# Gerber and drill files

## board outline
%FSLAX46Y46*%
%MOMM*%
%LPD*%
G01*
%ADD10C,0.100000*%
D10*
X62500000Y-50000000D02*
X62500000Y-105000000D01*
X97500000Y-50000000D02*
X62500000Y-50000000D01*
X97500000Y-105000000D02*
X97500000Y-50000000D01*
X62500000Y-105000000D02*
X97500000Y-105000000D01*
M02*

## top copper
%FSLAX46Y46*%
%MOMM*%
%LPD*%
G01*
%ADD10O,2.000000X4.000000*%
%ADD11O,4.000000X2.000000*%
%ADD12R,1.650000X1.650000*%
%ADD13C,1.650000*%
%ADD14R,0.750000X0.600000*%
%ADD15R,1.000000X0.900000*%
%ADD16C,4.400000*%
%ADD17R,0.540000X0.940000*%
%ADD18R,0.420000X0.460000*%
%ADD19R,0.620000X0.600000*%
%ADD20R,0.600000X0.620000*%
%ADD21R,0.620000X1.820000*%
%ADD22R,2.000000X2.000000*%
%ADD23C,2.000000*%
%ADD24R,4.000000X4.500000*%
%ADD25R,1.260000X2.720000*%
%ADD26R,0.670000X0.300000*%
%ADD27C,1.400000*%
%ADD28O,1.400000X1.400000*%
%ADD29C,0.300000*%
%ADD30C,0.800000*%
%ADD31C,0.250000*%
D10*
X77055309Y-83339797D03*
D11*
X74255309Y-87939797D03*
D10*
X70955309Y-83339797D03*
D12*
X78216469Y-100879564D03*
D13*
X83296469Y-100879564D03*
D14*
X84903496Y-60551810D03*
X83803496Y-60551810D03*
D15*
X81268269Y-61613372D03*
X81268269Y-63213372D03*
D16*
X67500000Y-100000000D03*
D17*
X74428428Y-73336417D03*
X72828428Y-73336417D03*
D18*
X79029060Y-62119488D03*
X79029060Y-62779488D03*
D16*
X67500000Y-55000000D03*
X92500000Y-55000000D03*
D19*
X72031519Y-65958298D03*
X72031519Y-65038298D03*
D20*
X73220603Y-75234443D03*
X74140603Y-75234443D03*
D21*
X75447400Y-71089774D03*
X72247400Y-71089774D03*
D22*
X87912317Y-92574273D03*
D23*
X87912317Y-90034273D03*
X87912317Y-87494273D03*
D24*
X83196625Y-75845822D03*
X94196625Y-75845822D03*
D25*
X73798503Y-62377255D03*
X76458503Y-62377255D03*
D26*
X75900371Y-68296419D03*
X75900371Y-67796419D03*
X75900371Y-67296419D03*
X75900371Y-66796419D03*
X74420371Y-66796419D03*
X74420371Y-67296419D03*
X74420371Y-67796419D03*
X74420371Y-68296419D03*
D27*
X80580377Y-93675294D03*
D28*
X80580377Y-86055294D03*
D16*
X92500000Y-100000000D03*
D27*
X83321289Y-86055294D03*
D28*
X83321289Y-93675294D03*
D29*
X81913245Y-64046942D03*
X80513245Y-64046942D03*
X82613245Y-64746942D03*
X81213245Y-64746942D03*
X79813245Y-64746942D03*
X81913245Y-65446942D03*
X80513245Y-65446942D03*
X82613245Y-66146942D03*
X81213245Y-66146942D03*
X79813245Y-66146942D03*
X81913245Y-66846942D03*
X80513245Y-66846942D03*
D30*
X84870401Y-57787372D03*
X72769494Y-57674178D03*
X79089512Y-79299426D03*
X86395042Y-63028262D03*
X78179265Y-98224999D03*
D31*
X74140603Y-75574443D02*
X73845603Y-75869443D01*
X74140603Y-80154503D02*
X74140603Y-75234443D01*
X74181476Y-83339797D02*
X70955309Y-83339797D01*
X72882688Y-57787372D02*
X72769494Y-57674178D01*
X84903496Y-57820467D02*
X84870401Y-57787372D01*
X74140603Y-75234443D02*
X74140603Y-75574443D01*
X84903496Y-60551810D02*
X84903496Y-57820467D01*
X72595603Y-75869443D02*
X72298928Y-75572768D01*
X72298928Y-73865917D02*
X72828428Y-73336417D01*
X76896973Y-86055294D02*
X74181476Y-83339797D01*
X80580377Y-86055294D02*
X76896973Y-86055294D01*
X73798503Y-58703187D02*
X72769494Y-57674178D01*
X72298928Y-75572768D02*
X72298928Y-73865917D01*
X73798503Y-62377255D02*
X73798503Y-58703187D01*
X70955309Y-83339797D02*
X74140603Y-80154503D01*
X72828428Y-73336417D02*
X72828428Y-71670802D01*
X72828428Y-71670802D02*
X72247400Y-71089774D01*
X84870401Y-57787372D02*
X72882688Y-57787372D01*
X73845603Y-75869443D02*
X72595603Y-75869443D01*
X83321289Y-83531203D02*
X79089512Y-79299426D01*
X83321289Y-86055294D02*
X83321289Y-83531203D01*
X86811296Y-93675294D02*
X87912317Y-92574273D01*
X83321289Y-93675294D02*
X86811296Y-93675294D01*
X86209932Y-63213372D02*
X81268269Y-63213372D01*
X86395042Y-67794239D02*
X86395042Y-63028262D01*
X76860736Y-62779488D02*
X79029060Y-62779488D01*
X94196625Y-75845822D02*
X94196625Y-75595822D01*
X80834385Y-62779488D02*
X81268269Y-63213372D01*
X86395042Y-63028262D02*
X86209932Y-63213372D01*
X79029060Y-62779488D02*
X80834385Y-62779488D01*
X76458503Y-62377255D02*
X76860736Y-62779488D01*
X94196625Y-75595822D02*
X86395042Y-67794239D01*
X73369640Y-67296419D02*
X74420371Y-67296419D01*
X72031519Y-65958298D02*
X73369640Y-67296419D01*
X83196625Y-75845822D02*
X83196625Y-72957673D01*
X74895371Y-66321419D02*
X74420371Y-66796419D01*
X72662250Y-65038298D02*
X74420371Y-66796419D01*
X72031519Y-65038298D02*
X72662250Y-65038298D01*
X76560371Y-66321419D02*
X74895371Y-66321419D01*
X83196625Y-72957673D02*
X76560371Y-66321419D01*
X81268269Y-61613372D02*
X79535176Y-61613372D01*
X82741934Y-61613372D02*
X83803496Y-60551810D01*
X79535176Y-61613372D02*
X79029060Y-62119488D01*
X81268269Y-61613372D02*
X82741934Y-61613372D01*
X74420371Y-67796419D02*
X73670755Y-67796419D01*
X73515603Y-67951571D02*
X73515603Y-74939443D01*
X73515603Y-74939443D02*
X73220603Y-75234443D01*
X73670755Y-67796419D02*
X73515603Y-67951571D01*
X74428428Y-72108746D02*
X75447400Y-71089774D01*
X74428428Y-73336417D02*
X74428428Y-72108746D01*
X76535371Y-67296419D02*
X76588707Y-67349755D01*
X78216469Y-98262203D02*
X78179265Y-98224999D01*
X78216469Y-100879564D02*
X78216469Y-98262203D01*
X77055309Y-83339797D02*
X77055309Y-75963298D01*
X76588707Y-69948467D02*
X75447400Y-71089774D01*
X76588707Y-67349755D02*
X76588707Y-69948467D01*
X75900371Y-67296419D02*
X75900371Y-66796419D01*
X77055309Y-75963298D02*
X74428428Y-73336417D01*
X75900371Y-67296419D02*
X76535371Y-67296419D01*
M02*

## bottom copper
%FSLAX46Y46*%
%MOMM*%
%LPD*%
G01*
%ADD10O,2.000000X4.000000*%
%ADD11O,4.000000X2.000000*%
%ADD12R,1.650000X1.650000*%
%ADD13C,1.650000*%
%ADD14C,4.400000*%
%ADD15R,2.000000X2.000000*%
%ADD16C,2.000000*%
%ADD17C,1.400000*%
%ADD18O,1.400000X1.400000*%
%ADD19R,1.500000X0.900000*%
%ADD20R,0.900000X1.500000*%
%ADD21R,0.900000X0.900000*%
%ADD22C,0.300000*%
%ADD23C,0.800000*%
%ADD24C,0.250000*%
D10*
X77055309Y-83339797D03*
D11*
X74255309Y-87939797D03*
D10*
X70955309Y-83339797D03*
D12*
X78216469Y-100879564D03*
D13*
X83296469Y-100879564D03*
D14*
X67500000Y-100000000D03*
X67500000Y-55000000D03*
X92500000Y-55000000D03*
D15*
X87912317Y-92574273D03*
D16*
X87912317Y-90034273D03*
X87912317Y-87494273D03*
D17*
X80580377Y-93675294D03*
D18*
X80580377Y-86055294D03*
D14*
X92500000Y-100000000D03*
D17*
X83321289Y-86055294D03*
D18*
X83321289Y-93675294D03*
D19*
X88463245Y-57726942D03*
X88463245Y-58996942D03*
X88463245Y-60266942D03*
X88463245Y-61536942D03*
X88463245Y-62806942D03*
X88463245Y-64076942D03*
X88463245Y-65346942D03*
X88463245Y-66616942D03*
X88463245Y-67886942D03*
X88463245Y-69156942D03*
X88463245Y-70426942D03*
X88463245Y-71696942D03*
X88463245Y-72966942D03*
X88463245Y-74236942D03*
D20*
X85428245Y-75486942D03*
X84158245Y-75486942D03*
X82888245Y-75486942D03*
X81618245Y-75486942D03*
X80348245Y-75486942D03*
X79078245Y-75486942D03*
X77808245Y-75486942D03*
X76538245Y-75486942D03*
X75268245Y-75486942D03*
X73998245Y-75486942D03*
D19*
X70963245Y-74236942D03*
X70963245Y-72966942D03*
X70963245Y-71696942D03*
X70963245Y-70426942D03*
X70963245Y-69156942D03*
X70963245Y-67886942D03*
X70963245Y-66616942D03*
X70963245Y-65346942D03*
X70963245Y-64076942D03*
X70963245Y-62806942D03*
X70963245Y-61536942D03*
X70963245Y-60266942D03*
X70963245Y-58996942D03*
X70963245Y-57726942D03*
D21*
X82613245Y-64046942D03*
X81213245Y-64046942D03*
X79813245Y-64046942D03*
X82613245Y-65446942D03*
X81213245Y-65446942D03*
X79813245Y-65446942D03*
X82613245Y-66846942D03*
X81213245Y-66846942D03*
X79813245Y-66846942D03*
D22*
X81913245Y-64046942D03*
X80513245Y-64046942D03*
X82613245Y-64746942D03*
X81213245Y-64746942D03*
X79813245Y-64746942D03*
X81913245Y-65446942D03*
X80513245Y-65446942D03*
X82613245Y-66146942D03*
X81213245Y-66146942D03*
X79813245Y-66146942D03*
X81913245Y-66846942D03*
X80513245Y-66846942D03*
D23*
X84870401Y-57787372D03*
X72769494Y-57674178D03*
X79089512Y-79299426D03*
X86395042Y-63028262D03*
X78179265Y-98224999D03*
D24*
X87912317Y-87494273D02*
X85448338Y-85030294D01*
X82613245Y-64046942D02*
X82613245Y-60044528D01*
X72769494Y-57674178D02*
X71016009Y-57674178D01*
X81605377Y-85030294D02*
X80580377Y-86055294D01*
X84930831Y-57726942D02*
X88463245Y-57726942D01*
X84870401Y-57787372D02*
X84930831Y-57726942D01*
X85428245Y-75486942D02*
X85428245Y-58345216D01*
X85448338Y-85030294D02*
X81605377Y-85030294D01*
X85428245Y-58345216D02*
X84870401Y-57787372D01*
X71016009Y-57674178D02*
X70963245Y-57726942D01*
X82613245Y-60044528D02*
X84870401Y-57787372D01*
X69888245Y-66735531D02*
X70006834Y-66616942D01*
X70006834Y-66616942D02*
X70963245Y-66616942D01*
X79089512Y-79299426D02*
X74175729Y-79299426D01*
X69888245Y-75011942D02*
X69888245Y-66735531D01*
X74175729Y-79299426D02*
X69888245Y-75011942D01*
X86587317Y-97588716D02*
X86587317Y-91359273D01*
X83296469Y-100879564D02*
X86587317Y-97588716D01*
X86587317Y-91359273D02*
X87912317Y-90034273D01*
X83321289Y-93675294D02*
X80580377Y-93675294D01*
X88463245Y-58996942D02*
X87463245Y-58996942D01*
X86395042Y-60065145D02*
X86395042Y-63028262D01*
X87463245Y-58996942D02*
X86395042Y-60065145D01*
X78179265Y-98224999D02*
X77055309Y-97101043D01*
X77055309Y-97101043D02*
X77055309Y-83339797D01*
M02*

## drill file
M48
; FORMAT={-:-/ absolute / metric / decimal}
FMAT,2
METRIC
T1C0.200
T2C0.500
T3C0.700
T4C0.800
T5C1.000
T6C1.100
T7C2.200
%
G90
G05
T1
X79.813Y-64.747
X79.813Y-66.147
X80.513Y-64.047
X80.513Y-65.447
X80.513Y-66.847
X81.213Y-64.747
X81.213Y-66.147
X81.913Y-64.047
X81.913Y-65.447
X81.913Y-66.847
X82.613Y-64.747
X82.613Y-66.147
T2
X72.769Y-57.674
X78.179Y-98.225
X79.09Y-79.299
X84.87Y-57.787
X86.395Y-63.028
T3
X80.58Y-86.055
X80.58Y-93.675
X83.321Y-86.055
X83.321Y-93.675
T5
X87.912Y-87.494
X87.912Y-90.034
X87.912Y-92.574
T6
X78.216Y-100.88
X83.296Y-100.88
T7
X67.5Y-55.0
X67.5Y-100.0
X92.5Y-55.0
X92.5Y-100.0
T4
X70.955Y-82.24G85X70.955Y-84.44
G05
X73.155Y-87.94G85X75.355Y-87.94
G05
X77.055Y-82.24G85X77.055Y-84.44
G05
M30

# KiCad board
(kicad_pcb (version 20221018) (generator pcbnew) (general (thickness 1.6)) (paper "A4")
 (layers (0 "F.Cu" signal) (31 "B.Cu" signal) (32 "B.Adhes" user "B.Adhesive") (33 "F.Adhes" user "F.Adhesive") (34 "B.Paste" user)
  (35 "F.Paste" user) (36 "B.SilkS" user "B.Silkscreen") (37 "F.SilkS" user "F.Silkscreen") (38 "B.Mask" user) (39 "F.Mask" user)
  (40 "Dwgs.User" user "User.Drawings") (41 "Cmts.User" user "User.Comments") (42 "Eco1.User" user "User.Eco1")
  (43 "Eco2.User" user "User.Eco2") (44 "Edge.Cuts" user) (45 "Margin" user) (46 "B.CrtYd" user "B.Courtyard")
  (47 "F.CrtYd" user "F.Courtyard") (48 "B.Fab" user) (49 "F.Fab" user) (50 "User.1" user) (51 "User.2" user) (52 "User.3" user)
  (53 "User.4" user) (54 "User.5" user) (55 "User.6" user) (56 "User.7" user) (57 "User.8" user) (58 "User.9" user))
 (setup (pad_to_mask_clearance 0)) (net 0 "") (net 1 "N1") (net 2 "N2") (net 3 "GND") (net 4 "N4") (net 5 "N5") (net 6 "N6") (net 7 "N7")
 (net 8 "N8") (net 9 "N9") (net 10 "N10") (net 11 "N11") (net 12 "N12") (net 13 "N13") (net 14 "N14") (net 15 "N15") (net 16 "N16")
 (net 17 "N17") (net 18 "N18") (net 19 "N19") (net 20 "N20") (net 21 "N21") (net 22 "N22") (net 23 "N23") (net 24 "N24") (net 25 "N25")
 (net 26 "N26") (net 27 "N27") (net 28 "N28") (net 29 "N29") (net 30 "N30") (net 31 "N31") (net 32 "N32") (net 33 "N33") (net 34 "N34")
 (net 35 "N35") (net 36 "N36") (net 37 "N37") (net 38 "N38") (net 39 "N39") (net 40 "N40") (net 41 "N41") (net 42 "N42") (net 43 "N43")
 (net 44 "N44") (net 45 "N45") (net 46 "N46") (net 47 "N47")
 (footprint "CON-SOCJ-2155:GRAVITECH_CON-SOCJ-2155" (layer "F.Cu") (at 70.955309 83.339797)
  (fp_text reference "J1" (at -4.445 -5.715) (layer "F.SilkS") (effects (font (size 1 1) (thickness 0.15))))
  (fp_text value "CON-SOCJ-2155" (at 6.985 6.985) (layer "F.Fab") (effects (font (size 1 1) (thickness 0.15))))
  (pad "1" thru_hole oval (at 6.1 0) (size 2 4) (drill oval 0.8 3) (layers "*.Cu" "*.Mask") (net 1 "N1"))
  (pad "2" thru_hole oval (at 3.3 4.6) (size 4 2) (drill oval 3 0.8) (layers "*.Cu" "*.Mask") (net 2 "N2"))
  (pad "3" thru_hole oval (at 0 0) (size 2 4) (drill oval 0.8 3) (layers "*.Cu" "*.Mask") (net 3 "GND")))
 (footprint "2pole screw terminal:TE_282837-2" (layer "F.Cu") (at 80.756469 100.879564)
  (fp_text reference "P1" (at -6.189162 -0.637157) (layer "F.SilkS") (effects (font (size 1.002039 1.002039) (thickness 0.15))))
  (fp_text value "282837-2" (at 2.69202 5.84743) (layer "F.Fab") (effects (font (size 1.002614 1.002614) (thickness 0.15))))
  (pad "1" thru_hole rect (at -2.54 0) (size 1.65 1.65) (drill 1.1) (layers "*.Cu" "*.Mask") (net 1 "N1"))
  (pad "2" thru_hole circle (at 2.54 0) (size 1.65 1.65) (drill 1.1) (layers "*.Cu" "*.Mask") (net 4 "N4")))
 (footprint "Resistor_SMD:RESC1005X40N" (layer "F.Cu") (at 84.353496 60.55181 180)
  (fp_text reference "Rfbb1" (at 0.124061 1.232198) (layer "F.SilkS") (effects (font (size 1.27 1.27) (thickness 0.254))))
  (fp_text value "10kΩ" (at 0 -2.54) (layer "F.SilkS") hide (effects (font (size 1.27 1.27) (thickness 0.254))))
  (pad "1" smd rect (at -0.55 0 270) (size 0.6 0.75) (layers "F.Cu" "F.Paste" "F.Mask") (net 3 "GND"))
  (pad "2" smd rect (at 0.55 0 270) (size 0.6 0.75) (layers "F.Cu" "F.Paste" "F.Mask") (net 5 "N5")))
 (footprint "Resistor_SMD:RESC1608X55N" (layer "F.Cu") (at 81.268269 62.413372 -90)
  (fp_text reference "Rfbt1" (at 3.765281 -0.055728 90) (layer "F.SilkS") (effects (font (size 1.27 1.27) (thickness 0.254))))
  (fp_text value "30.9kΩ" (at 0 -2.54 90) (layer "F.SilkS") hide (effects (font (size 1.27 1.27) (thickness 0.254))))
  (pad "1" smd rect (at -0.8 0 270) (size 0.9 1) (layers "F.Cu" "F.Paste" "F.Mask") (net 5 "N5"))
  (pad "2" smd rect (at 0.8 0 270) (size 0.9 1) (layers "F.Cu" "F.Paste" "F.Mask") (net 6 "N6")))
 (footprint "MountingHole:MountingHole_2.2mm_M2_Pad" (layer "F.Cu") (at 67.5 100)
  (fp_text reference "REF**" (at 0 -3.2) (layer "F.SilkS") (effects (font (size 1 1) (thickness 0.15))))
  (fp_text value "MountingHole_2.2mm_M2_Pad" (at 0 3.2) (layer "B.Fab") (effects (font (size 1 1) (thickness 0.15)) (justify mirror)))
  (pad "1" thru_hole circle (at 0 0) (size 4.4 4.4) (drill 2.2) (layers "*.Cu" "*.Mask")))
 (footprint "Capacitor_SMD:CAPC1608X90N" (layer "F.Cu") (at 73.628428 73.336417 180)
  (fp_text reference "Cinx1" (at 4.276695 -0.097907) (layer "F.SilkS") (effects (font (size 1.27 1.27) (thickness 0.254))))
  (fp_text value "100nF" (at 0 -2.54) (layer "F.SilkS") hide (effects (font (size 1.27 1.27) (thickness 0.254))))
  (pad "1" smd rect (at -0.8 0 180) (size 0.54 0.94) (layers "F.Cu" "F.Paste" "F.Mask") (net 1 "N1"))
  (pad "2" smd rect (at 0.8 0 180) (size 0.54 0.94) (layers "F.Cu" "F.Paste" "F.Mask") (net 3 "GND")))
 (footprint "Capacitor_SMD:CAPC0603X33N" (layer "F.Cu") (at 79.02906 62.449488 -90)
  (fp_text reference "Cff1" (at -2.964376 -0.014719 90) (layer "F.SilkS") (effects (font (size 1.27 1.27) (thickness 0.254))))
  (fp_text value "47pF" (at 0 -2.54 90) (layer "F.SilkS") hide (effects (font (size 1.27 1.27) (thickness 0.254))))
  (pad "1" smd rect (at -0.33 0) (size 0.42 0.46) (layers "F.Cu" "F.Paste" "F.Mask") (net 5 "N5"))
  (pad "2" smd rect (at 0.33 0) (size 0.42 0.46) (layers "F.Cu" "F.Paste" "F.Mask") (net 6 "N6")))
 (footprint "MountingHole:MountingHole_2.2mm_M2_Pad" (layer "F.Cu") (at 67.5 55)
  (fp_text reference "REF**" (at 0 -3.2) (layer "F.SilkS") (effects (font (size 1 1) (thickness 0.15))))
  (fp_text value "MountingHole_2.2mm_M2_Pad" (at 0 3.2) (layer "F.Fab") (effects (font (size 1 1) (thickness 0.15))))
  (pad "1" thru_hole circle (at 0 0) (size 4.4 4.4) (drill 2.2) (layers "*.Cu" "*.Mask")))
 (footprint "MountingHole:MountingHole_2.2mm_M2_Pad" (layer "F.Cu") (at 92.5 55)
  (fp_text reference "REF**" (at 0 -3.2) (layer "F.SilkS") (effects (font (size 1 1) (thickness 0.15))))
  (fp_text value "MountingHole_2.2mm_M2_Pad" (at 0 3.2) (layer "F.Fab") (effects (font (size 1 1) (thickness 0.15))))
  (pad "1" thru_hole circle (at 0 0) (size 4.4 4.4) (drill 2.2) (layers "*.Cu" "*.Mask")))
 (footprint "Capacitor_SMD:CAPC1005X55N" (layer "F.Cu") (at 72.031519 65.498298 90)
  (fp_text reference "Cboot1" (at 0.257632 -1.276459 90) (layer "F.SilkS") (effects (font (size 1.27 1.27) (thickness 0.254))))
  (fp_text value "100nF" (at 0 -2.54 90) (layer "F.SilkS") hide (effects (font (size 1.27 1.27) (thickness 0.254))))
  (pad "1" smd rect (at -0.46 0 90) (size 0.6 0.62) (layers "F.Cu" "F.Paste" "F.Mask") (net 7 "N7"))
  (pad "2" smd rect (at 0.46 0 90) (size 0.6 0.62) (layers "F.Cu" "F.Paste" "F.Mask") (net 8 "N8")))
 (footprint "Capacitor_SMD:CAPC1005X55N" (layer "F.Cu") (at 73.680603 75.234443)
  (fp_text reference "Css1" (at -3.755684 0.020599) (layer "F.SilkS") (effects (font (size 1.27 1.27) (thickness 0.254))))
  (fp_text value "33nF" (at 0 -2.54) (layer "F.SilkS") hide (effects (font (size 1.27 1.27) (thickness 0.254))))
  (pad "1" smd rect (at -0.46 0) (size 0.6 0.62) (layers "F.Cu" "F.Paste" "F.Mask") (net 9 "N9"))
  (pad "2" smd rect (at 0.46 0) (size 0.6 0.62) (layers "F.Cu" "F.Paste" "F.Mask") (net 3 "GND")))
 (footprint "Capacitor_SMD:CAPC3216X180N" (layer "F.Cu") (at 73.8474 71.089774 180)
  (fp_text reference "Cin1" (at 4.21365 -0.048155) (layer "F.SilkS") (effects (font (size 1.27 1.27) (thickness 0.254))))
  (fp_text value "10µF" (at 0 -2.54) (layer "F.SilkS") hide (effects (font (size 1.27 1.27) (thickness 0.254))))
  (pad "1" smd rect (at -1.6 0 180) (size 0.62 1.82) (layers "F.Cu" "F.Paste" "F.Mask") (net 1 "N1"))
  (pad "2" smd rect (at 1.6 0 180) (size 0.62 1.82) (layers "F.Cu" "F.Paste" "F.Mask") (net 3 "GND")))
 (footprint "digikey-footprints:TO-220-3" (layer "F.Cu") (at 87.912317 92.574273 90)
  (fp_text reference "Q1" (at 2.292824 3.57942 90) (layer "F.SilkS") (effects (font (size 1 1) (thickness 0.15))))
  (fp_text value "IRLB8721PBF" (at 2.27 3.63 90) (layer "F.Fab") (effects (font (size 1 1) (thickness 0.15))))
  (pad "1" thru_hole rect (at 0 0 90) (size 2 2) (drill 1) (layers "*.Cu" "*.Mask") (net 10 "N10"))
  (pad "2" thru_hole circle (at 2.54 0 90) (size 2 2) (drill 1) (layers "*.Cu" "*.Mask") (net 4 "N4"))
  (pad "3" thru_hole circle (at 5.08 0 90) (size 2 2) (drill 1) (layers "*.Cu" "*.Mask") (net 3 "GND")))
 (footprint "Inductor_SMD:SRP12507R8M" (layer "F.Cu") (at 88.696625 75.845822)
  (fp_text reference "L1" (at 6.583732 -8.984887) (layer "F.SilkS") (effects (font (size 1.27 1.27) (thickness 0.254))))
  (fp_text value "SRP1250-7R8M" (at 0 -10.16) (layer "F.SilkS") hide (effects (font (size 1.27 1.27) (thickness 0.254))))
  (pad "1" smd rect (at -5.5 0) (size 4 4.5) (layers "F.Cu" "F.Paste" "F.Mask") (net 8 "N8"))
  (pad "2" smd rect (at 5.5 0) (size 4 4.5) (layers "F.Cu" "F.Paste" "F.Mask") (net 6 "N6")))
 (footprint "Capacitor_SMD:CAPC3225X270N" (layer "F.Cu") (at 75.128503 62.377255)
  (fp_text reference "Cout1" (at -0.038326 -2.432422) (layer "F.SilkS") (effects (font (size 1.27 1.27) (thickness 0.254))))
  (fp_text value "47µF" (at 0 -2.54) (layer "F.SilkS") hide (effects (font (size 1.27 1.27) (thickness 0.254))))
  (pad "1" smd rect (at -1.33 0) (size 1.26 2.72) (layers "F.Cu" "F.Paste" "F.Mask") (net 3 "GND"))
  (pad "2" smd rect (at 1.33 0) (size 1.26 2.72) (layers "F.Cu" "F.Paste" "F.Mask") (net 6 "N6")))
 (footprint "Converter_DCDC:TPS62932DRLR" (layer "F.Cu") (at 75.160371 67.546419 180)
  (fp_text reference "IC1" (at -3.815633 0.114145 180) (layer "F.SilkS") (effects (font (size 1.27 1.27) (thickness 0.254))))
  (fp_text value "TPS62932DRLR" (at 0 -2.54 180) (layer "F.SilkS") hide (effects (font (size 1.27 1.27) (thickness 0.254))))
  (pad "1" smd rect (at -0.74 -0.75 270) (size 0.3 0.67) (layers "F.Cu" "F.Paste" "F.Mask") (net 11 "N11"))
  (pad "2" smd rect (at -0.74 -0.25 270) (size 0.3 0.67) (layers "F.Cu" "F.Paste" "F.Mask") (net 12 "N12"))
  (pad "3" smd rect (at -0.74 0.25 270) (size 0.3 0.67) (layers "F.Cu" "F.Paste" "F.Mask") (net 1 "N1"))
  (pad "4" smd rect (at -0.74 0.75 270) (size 0.3 0.67) (layers "F.Cu" "F.Paste" "F.Mask") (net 1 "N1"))
  (pad "5" smd rect (at 0.74 0.75 270) (size 0.3 0.67) (layers "F.Cu" "F.Paste" "F.Mask") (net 8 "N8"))
  (pad "6" smd rect (at 0.74 0.25 270) (size 0.3 0.67) (layers "F.Cu" "F.Paste" "F.Mask") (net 7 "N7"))
  (pad "7" smd rect (at 0.74 -0.25 270) (size 0.3 0.67) (layers "F.Cu" "F.Paste" "F.Mask") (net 9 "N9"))
  (pad "8" smd rect (at 0.74 -0.75 270) (size 0.3 0.67) (layers "F.Cu" "F.Paste" "F.Mask") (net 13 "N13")))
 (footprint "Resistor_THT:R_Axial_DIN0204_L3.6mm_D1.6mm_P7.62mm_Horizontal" (layer "F.Cu") (at 80.580377 93.675294 90)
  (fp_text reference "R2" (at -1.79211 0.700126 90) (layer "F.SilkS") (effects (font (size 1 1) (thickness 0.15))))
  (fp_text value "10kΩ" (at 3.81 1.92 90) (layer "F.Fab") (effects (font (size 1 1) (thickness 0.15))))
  (pad "1" thru_hole circle (at 0 0 90) (size 1.4 1.4) (drill 0.7) (layers "*.Cu" "*.Mask") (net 10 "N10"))
  (pad "2" thru_hole oval (at 7.62 0 90) (size 1.4 1.4) (drill 0.7) (layers "*.Cu" "*.Mask") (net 3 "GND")))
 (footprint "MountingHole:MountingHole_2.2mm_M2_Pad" (layer "F.Cu") (at 92.5 100)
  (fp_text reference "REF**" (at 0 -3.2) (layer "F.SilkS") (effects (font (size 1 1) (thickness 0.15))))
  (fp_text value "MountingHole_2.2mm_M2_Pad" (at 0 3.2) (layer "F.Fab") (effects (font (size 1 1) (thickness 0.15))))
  (pad "1" thru_hole circle (at 0 0) (size 4.4 4.4) (drill 2.2) (layers "*.Cu" "*.Mask")))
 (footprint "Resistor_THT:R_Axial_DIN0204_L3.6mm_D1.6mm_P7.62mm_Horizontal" (layer "F.Cu") (at 83.321289 86.055294 -90)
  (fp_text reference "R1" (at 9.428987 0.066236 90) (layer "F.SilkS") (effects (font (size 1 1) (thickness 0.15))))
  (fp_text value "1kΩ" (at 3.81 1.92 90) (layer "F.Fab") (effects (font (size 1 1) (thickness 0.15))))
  (pad "1" thru_hole circle (at 0 0 270) (size 1.4 1.4) (drill 0.7) (layers "*.Cu" "*.Mask") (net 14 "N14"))
  (pad "2" thru_hole oval (at 7.62 0 270) (size 1.4 1.4) (drill 0.7) (layers "*.Cu" "*.Mask") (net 10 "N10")))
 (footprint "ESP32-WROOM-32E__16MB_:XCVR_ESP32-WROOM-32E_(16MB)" (layer "B.Cu") (at 79.713245 62.986942 180)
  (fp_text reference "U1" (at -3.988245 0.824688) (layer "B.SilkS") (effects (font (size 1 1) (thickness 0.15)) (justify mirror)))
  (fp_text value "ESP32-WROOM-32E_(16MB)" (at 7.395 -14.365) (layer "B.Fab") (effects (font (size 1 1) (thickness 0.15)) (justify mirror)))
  (pad "1" smd rect (at -8.75 5.26 180) (size 1.5 0.9) (layers "B.Cu" "B.Paste" "B.Mask") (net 3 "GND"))
  (pad "2" smd rect (at -8.75 3.99 180) (size 1.5 0.9) (layers "B.Cu" "B.Paste" "B.Mask") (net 6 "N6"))
  (pad "3" smd rect (at -8.75 2.72 180) (size 1.5 0.9) (layers "B.Cu" "B.Paste" "B.Mask") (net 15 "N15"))
  (pad "4" smd rect (at -8.75 1.45 180) (size 1.5 0.9) (layers "B.Cu" "B.Paste" "B.Mask") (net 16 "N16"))
  (pad "5" smd rect (at -8.75 0.18 180) (size 1.5 0.9) (layers "B.Cu" "B.Paste" "B.Mask") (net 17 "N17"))
  (pad "6" smd rect (at -8.75 -1.09 180) (size 1.5 0.9) (layers "B.Cu" "B.Paste" "B.Mask") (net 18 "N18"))
  (pad "7" smd rect (at -8.75 -2.36 180) (size 1.5 0.9) (layers "B.Cu" "B.Paste" "B.Mask") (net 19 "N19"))
  (pad "8" smd rect (at -8.75 -3.63 180) (size 1.5 0.9) (layers "B.Cu" "B.Paste" "B.Mask") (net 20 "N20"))
  (pad "9" smd rect (at -8.75 -4.9 180) (size 1.5 0.9) (layers "B.Cu" "B.Paste" "B.Mask") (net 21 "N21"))
  (pad "10" smd rect (at -8.75 -6.17 180) (size 1.5 0.9) (layers "B.Cu" "B.Paste" "B.Mask") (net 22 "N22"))
  (pad "11" smd rect (at -8.75 -7.44 180) (size 1.5 0.9) (layers "B.Cu" "B.Paste" "B.Mask") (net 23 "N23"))
  (pad "12" smd rect (at -8.75 -8.71 180) (size 1.5 0.9) (layers "B.Cu" "B.Paste" "B.Mask") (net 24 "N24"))
  (pad "13" smd rect (at -8.75 -9.98 180) (size 1.5 0.9) (layers "B.Cu" "B.Paste" "B.Mask") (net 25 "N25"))
  (pad "14" smd rect (at -8.75 -11.25 180) (size 1.5 0.9) (layers "B.Cu" "B.Paste" "B.Mask") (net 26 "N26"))
  (pad "15" smd rect (at -5.715 -12.5 180) (size 0.9 1.5) (layers "B.Cu" "B.Paste" "B.Mask") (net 3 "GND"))
  (pad "16" smd rect (at -4.445 -12.5 180) (size 0.9 1.5) (layers "B.Cu" "B.Paste" "B.Mask") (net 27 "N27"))
  (pad "17" smd rect (at -3.175 -12.5 180) (size 0.9 1.5) (layers "B.Cu" "B.Paste" "B.Mask") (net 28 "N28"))
  (pad "18" smd rect (at -1.905 -12.5 180) (size 0.9 1.5) (layers "B.Cu" "B.Paste" "B.Mask") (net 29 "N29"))
  (pad "19" smd rect (at -0.635 -12.5 180) (size 0.9 1.5) (layers "B.Cu" "B.Paste" "B.Mask") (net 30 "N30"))
  (pad "20" smd rect (at 0.635 -12.5 180) (size 0.9 1.5) (layers "B.Cu" "B.Paste" "B.Mask") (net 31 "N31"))
  (pad "21" smd rect (at 1.905 -12.5 180) (size 0.9 1.5) (layers "B.Cu" "B.Paste" "B.Mask") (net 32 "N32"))
  (pad "22" smd rect (at 3.175 -12.5 180) (size 0.9 1.5) (layers "B.Cu" "B.Paste" "B.Mask") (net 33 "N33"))
  (pad "23" smd rect (at 4.445 -12.5 180) (size 0.9 1.5) (layers "B.Cu" "B.Paste" "B.Mask") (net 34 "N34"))
  (pad "24" smd rect (at 5.715 -12.5 180) (size 0.9 1.5) (layers "B.Cu" "B.Paste" "B.Mask") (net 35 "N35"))
  (pad "25" smd rect (at 8.75 -11.25 180) (size 1.5 0.9) (layers "B.Cu" "B.Paste" "B.Mask") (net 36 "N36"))
  (pad "26" smd rect (at 8.75 -9.98 180) (size 1.5 0.9) (layers "B.Cu" "B.Paste" "B.Mask") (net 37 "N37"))
  (pad "27" smd rect (at 8.75 -8.71 180) (size 1.5 0.9) (layers "B.Cu" "B.Paste" "B.Mask") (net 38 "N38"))
  (pad "28" smd rect (at 8.75 -7.44 180) (size 1.5 0.9) (layers "B.Cu" "B.Paste" "B.Mask") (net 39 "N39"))
  (pad "29" smd rect (at 8.75 -6.17 180) (size 1.5 0.9) (layers "B.Cu" "B.Paste" "B.Mask") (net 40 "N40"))
  (pad "30" smd rect (at 8.75 -4.9 180) (size 1.5 0.9) (layers "B.Cu" "B.Paste" "B.Mask") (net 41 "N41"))
  (pad "31" smd rect (at 8.75 -3.63 180) (size 1.5 0.9) (layers "B.Cu" "B.Paste" "B.Mask") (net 14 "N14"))
  (pad "32" smd rect (at 8.75 -2.36 180) (size 1.5 0.9) (layers "B.Cu" "B.Paste" "B.Mask") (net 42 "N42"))
  (pad "33" smd rect (at 8.75 -1.09 180) (size 1.5 0.9) (layers "B.Cu" "B.Paste" "B.Mask") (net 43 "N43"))
  (pad "34" smd rect (at 8.75 0.18 180) (size 1.5 0.9) (layers "B.Cu" "B.Paste" "B.Mask") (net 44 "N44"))
  (pad "35" smd rect (at 8.75 1.45 180) (size 1.5 0.9) (layers "B.Cu" "B.Paste" "B.Mask") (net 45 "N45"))
  (pad "36" smd rect (at 8.75 2.72 180) (size 1.5 0.9) (layers "B.Cu" "B.Paste" "B.Mask") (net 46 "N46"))
  (pad "37" smd rect (at 8.75 3.99 180) (size 1.5 0.9) (layers "B.Cu" "B.Paste" "B.Mask") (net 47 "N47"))
  (pad "38" smd rect (at 8.75 5.26 180) (size 1.5 0.9) (layers "B.Cu" "B.Paste" "B.Mask") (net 3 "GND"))
  (pad "39_1" smd rect (at -2.9 -1.06 180) (size 0.9 0.9) (layers "B.Cu" "B.Paste" "B.Mask") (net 3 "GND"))
  (pad "39_2" smd rect (at -1.5 -1.06 180) (size 0.9 0.9) (layers "B.Cu" "B.Paste" "B.Mask") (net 3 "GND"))
  (pad "39_3" smd rect (at -0.1 -1.06 180) (size 0.9 0.9) (layers "B.Cu" "B.Paste" "B.Mask") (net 3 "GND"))
  (pad "39_4" smd rect (at -2.9 -2.46 180) (size 0.9 0.9) (layers "B.Cu" "B.Paste" "B.Mask") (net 3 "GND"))
  (pad "39_5" smd rect (at -1.5 -2.46 180) (size 0.9 0.9) (layers "B.Cu" "B.Paste" "B.Mask") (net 3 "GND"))
  (pad "39_6" smd rect (at -0.1 -2.46 180) (size 0.9 0.9) (layers "B.Cu" "B.Paste" "B.Mask") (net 3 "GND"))
  (pad "39_7" smd rect (at -2.9 -3.86 180) (size 0.9 0.9) (layers "B.Cu" "B.Paste" "B.Mask") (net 3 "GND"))
  (pad "39_8" smd rect (at -1.5 -3.86 180) (size 0.9 0.9) (layers "B.Cu" "B.Paste" "B.Mask") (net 3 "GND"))
  (pad "39_9" smd rect (at -0.1 -3.86 180) (size 0.9 0.9) (layers "B.Cu" "B.Paste" "B.Mask") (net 3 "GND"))
  (pad "39_10" thru_hole circle (at -2.2 -1.06 180) (size 0.3 0.3) (drill 0.2) (layers "*.Cu"))
  (pad "39_11" thru_hole circle (at -0.8 -1.06 180) (size 0.3 0.3) (drill 0.2) (layers "*.Cu"))
  (pad "39_12" thru_hole circle (at -2.9 -1.76 180) (size 0.3 0.3) (drill 0.2) (layers "*.Cu"))
  (pad "39_13" thru_hole circle (at -1.5 -1.76 180) (size 0.3 0.3) (drill 0.2) (layers "*.Cu"))
  (pad "39_14" thru_hole circle (at -0.1 -1.76 180) (size 0.3 0.3) (drill 0.2) (layers "*.Cu"))
  (pad "39_15" thru_hole circle (at -2.2 -2.46 180) (size 0.3 0.3) (drill 0.2) (layers "*.Cu"))
  (pad "39_16" thru_hole circle (at -0.8 -2.46 180) (size 0.3 0.3) (drill 0.2) (layers "*.Cu"))
  (pad "39_17" thru_hole circle (at -2.9 -3.16 180) (size 0.3 0.3) (drill 0.2) (layers "*.Cu"))
  (pad "39_18" thru_hole circle (at -1.5 -3.16 180) (size 0.3 0.3) (drill 0.2) (layers "*.Cu"))
  (pad "39_19" thru_hole circle (at -0.1 -3.16 180) (size 0.3 0.3) (drill 0.2) (layers "*.Cu"))
  (pad "39_20" thru_hole circle (at -2.2 -3.86 180) (size 0.3 0.3) (drill 0.2) (layers "*.Cu"))
  (pad "39_21" thru_hole circle (at -0.8 -3.86 180) (size 0.3 0.3) (drill 0.2) (layers "*.Cu"))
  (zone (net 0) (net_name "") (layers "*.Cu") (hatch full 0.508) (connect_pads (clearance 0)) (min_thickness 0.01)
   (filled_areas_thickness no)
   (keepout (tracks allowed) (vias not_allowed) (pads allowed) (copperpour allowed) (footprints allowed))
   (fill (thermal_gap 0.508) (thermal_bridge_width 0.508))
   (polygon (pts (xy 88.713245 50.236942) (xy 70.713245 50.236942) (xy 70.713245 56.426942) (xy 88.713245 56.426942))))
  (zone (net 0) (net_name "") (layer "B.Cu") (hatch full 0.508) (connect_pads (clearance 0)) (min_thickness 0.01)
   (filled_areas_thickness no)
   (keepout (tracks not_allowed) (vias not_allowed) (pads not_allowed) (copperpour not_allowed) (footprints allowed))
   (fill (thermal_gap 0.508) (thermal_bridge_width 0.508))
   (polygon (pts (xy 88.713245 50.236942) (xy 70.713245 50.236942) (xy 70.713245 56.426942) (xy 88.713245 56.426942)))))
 (gr_line (start 62.5 50) (end 62.5 105) (stroke (width 0.1) (type default)) (layer "Edge.Cuts"))
 (gr_line (start 97.5 50) (end 62.5 50) (stroke (width 0.1) (type default)) (layer "Edge.Cuts"))
 (gr_line (start 97.5 105) (end 97.5 50) (stroke (width 0.1) (type default)) (layer "Edge.Cuts"))
 (gr_line (start 62.5 105) (end 97.5 105) (stroke (width 0.1) (type default)) (layer "Edge.Cuts"))
 (segment (start 74.140603 75.574443) (end 73.845603 75.869443) (width 0.25) (layer "F.Cu") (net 3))
 (segment (start 74.140603 80.154503) (end 74.140603 75.234443) (width 0.25) (layer "F.Cu") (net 3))
 (segment (start 74.181476 83.339797) (end 70.955309 83.339797) (width 0.25) (layer "F.Cu") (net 3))
 (segment (start 72.882688 57.787372) (end 72.769494 57.674178) (width 0.25) (layer "F.Cu") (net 3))
 (segment (start 84.903496 57.820467) (end 84.870401 57.787372) (width 0.25) (layer "F.Cu") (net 3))
 (segment (start 74.140603 75.234443) (end 74.140603 75.574443) (width 0.25) (layer "F.Cu") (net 3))
 (segment (start 84.903496 60.55181) (end 84.903496 57.820467) (width 0.25) (layer "F.Cu") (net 3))
 (segment (start 72.595603 75.869443) (end 72.298928 75.572768) (width 0.25) (layer "F.Cu") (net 3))
 (segment (start 72.298928 73.865917) (end 72.828428 73.336417) (width 0.25) (layer "F.Cu") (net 3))
 (segment (start 76.896973 86.055294) (end 74.181476 83.339797) (width 0.25) (layer "F.Cu") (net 3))
 (segment (start 80.580377 86.055294) (end 76.896973 86.055294) (width 0.25) (layer "F.Cu") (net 3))
 (segment (start 73.798503 58.703187) (end 72.769494 57.674178) (width 0.25) (layer "F.Cu") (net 3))
 (segment (start 72.298928 75.572768) (end 72.298928 73.865917) (width 0.25) (layer "F.Cu") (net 3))
 (segment (start 73.798503 62.377255) (end 73.798503 58.703187) (width 0.25) (layer "F.Cu") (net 3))
 (segment (start 70.955309 83.339797) (end 74.140603 80.154503) (width 0.25) (layer "F.Cu") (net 3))
 (segment (start 72.828428 73.336417) (end 72.828428 71.670802) (width 0.25) (layer "F.Cu") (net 3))
 (segment (start 72.828428 71.670802) (end 72.2474 71.089774) (width 0.25) (layer "F.Cu") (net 3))
 (segment (start 84.870401 57.787372) (end 72.882688 57.787372) (width 0.25) (layer "F.Cu") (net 3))
 (segment (start 73.845603 75.869443) (end 72.595603 75.869443) (width 0.25) (layer "F.Cu") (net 3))
 (via (at 84.870401 57.787372) (size 0.8) (drill 0.5) (layers "F.Cu" "B.Cu") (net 3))
 (via (at 72.769494 57.674178) (size 0.8) (drill 0.5) (layers "F.Cu" "B.Cu") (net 3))
 (segment (start 87.912317 87.494273) (end 85.448338 85.030294) (width 0.25) (layer "B.Cu") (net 3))
 (segment (start 82.613245 64.046942) (end 82.613245 60.044528) (width 0.25) (layer "B.Cu") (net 3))
 (segment (start 72.769494 57.674178) (end 71.016009 57.674178) (width 0.25) (layer "B.Cu") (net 3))
 (segment (start 81.605377 85.030294) (end 80.580377 86.055294) (width 0.25) (layer "B.Cu") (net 3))
 (segment (start 84.930831 57.726942) (end 88.463245 57.726942) (width 0.25) (layer "B.Cu") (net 3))
 (segment (start 84.870401 57.787372) (end 84.930831 57.726942) (width 0.25) (layer "B.Cu") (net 3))
 (segment (start 85.428245 75.486942) (end 85.428245 58.345216) (width 0.25) (layer "B.Cu") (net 3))
 (segment (start 85.448338 85.030294) (end 81.605377 85.030294) (width 0.25) (layer "B.Cu") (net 3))
 (segment (start 85.428245 58.345216) (end 84.870401 57.787372) (width 0.25) (layer "B.Cu") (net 3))
 (segment (start 71.016009 57.674178) (end 70.963245 57.726942) (width 0.25) (layer "B.Cu") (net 3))
 (segment (start 82.613245 60.044528) (end 84.870401 57.787372) (width 0.25) (layer "B.Cu") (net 3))
 (segment (start 83.321289 83.531203) (end 79.089512 79.299426) (width 0.25) (layer "F.Cu") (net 14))
 (segment (start 83.321289 86.055294) (end 83.321289 83.531203) (width 0.25) (layer "F.Cu") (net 14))
 (via (at 79.089512 79.299426) (size 0.8) (drill 0.5) (layers "F.Cu" "B.Cu") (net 14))
 (segment (start 69.888245 66.735531) (end 70.006834 66.616942) (width 0.25) (layer "B.Cu") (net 14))
 (segment (start 70.006834 66.616942) (end 70.963245 66.616942) (width 0.25) (layer "B.Cu") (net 14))
 (segment (start 79.089512 79.299426) (end 74.175729 79.299426) (width 0.25) (layer "B.Cu") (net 14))
 (segment (start 69.888245 75.011942) (end 69.888245 66.735531) (width 0.25) (layer "B.Cu") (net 14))
 (segment (start 74.175729 79.299426) (end 69.888245 75.011942) (width 0.25) (layer "B.Cu") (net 14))
 (segment (start 86.587317 97.588716) (end 86.587317 91.359273) (width 0.25) (layer "B.Cu") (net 4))
 (segment (start 83.296469 100.879564) (end 86.587317 97.588716) (width 0.25) (layer "B.Cu") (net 4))
 (segment (start 86.587317 91.359273) (end 87.912317 90.034273) (width 0.25) (layer "B.Cu") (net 4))
 (segment (start 86.811296 93.675294) (end 87.912317 92.574273) (width 0.25) (layer "F.Cu") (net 10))
 (segment (start 83.321289 93.675294) (end 86.811296 93.675294) (width 0.25) (layer "F.Cu") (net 10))
 (segment (start 83.321289 93.675294) (end 80.580377 93.675294) (width 0.25) (layer "B.Cu") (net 10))
 (segment (start 86.209932 63.213372) (end 81.268269 63.213372) (width 0.25) (layer "F.Cu") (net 6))
 (segment (start 86.395042 67.794239) (end 86.395042 63.028262) (width 0.25) (layer "F.Cu") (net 6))
 (segment (start 76.860736 62.779488) (end 79.02906 62.779488) (width 0.25) (layer "F.Cu") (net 6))
 (segment (start 94.196625 75.845822) (end 94.196625 75.595822) (width 0.25) (layer "F.Cu") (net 6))
 (segment (start 80.834385 62.779488) (end 81.268269 63.213372) (width 0.25) (layer "F.Cu") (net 6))
 (segment (start 86.395042 63.028262) (end 86.209932 63.213372) (width 0.25) (layer "F.Cu") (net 6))
 (segment (start 79.02906 62.779488) (end 80.834385 62.779488) (width 0.25) (layer "F.Cu") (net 6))
 (segment (start 76.458503 62.377255) (end 76.860736 62.779488) (width 0.25) (layer "F.Cu") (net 6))
 (segment (start 94.196625 75.595822) (end 86.395042 67.794239) (width 0.25) (layer "F.Cu") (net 6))
 (via (at 86.395042 63.028262) (size 0.8) (drill 0.5) (layers "F.Cu" "B.Cu") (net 6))
 (segment (start 88.463245 58.996942) (end 87.463245 58.996942) (width 0.25) (layer "B.Cu") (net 6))
 (segment (start 86.395042 60.065145) (end 86.395042 63.028262) (width 0.25) (layer "B.Cu") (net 6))
 (segment (start 87.463245 58.996942) (end 86.395042 60.065145) (width 0.25) (layer "B.Cu") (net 6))
 (segment (start 73.36964 67.296419) (end 74.420371 67.296419) (width 0.25) (layer "F.Cu") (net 7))
 (segment (start 72.031519 65.958298) (end 73.36964 67.296419) (width 0.25) (layer "F.Cu") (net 7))
 (segment (start 83.196625 75.845822) (end 83.196625 72.957673) (width 0.25) (layer "F.Cu") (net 8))
 (segment (start 74.895371 66.321419) (end 74.420371 66.796419) (width 0.25) (layer "F.Cu") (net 8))
 (segment (start 72.66225 65.038298) (end 74.420371 66.796419) (width 0.25) (layer "F.Cu") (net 8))
 (segment (start 72.031519 65.038298) (end 72.66225 65.038298) (width 0.25) (layer "F.Cu") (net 8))
 (segment (start 76.560371 66.321419) (end 74.895371 66.321419) (width 0.25) (layer "F.Cu") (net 8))
 (segment (start 83.196625 72.957673) (end 76.560371 66.321419) (width 0.25) (layer "F.Cu") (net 8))
 (segment (start 81.268269 61.613372) (end 79.535176 61.613372) (width 0.25) (layer "F.Cu") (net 5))
 (segment (start 82.741934 61.613372) (end 83.803496 60.55181) (width 0.25) (layer "F.Cu") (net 5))
 (segment (start 79.535176 61.613372) (end 79.02906 62.119488) (width 0.25) (layer "F.Cu") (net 5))
 (segment (start 81.268269 61.613372) (end 82.741934 61.613372) (width 0.25) (layer "F.Cu") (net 5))
 (segment (start 74.420371 67.796419) (end 73.670755 67.796419) (width 0.25) (layer "F.Cu") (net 9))
 (segment (start 73.515603 67.951571) (end 73.515603 74.939443) (width 0.25) (layer "F.Cu") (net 9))
 (segment (start 73.515603 74.939443) (end 73.220603 75.234443) (width 0.25) (layer "F.Cu") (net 9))
 (segment (start 73.670755 67.796419) (end 73.515603 67.951571) (width 0.25) (layer "F.Cu") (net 9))
 (segment (start 74.428428 72.108746) (end 75.4474 71.089774) (width 0.25) (layer "F.Cu") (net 1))
 (segment (start 74.428428 73.336417) (end 74.428428 72.108746) (width 0.25) (layer "F.Cu") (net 1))
 (segment (start 76.535371 67.296419) (end 76.588707 67.349755) (width 0.25) (layer "F.Cu") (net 1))
 (segment (start 78.216469 98.262203) (end 78.179265 98.224999) (width 0.25) (layer "F.Cu") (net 1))
 (segment (start 78.216469 100.879564) (end 78.216469 98.262203) (width 0.25) (layer "F.Cu") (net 1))
 (segment (start 77.055309 83.339797) (end 77.055309 75.963298) (width 0.25) (layer "F.Cu") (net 1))
 (segment (start 76.588707 69.948467) (end 75.4474 71.089774) (width 0.25) (layer "F.Cu") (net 1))
 (segment (start 76.588707 67.349755) (end 76.588707 69.948467) (width 0.25) (layer "F.Cu") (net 1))
 (segment (start 75.900371 67.296419) (end 75.900371 66.796419) (width 0.25) (layer "F.Cu") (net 1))
 (segment (start 77.055309 75.963298) (end 74.428428 73.336417) (width 0.25) (layer "F.Cu") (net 1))
 (segment (start 75.900371 67.296419) (end 76.535371 67.296419) (width 0.25) (layer "F.Cu") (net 1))
 (via (at 78.179265 98.224999) (size 0.8) (drill 0.5) (layers "F.Cu" "B.Cu") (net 1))
 (segment (start 78.179265 98.224999) (end 77.055309 97.101043) (width 0.25) (layer "B.Cu") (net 1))
 (segment (start 77.055309 97.101043) (end 77.055309 83.339797) (width 0.25) (layer "B.Cu") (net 1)))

